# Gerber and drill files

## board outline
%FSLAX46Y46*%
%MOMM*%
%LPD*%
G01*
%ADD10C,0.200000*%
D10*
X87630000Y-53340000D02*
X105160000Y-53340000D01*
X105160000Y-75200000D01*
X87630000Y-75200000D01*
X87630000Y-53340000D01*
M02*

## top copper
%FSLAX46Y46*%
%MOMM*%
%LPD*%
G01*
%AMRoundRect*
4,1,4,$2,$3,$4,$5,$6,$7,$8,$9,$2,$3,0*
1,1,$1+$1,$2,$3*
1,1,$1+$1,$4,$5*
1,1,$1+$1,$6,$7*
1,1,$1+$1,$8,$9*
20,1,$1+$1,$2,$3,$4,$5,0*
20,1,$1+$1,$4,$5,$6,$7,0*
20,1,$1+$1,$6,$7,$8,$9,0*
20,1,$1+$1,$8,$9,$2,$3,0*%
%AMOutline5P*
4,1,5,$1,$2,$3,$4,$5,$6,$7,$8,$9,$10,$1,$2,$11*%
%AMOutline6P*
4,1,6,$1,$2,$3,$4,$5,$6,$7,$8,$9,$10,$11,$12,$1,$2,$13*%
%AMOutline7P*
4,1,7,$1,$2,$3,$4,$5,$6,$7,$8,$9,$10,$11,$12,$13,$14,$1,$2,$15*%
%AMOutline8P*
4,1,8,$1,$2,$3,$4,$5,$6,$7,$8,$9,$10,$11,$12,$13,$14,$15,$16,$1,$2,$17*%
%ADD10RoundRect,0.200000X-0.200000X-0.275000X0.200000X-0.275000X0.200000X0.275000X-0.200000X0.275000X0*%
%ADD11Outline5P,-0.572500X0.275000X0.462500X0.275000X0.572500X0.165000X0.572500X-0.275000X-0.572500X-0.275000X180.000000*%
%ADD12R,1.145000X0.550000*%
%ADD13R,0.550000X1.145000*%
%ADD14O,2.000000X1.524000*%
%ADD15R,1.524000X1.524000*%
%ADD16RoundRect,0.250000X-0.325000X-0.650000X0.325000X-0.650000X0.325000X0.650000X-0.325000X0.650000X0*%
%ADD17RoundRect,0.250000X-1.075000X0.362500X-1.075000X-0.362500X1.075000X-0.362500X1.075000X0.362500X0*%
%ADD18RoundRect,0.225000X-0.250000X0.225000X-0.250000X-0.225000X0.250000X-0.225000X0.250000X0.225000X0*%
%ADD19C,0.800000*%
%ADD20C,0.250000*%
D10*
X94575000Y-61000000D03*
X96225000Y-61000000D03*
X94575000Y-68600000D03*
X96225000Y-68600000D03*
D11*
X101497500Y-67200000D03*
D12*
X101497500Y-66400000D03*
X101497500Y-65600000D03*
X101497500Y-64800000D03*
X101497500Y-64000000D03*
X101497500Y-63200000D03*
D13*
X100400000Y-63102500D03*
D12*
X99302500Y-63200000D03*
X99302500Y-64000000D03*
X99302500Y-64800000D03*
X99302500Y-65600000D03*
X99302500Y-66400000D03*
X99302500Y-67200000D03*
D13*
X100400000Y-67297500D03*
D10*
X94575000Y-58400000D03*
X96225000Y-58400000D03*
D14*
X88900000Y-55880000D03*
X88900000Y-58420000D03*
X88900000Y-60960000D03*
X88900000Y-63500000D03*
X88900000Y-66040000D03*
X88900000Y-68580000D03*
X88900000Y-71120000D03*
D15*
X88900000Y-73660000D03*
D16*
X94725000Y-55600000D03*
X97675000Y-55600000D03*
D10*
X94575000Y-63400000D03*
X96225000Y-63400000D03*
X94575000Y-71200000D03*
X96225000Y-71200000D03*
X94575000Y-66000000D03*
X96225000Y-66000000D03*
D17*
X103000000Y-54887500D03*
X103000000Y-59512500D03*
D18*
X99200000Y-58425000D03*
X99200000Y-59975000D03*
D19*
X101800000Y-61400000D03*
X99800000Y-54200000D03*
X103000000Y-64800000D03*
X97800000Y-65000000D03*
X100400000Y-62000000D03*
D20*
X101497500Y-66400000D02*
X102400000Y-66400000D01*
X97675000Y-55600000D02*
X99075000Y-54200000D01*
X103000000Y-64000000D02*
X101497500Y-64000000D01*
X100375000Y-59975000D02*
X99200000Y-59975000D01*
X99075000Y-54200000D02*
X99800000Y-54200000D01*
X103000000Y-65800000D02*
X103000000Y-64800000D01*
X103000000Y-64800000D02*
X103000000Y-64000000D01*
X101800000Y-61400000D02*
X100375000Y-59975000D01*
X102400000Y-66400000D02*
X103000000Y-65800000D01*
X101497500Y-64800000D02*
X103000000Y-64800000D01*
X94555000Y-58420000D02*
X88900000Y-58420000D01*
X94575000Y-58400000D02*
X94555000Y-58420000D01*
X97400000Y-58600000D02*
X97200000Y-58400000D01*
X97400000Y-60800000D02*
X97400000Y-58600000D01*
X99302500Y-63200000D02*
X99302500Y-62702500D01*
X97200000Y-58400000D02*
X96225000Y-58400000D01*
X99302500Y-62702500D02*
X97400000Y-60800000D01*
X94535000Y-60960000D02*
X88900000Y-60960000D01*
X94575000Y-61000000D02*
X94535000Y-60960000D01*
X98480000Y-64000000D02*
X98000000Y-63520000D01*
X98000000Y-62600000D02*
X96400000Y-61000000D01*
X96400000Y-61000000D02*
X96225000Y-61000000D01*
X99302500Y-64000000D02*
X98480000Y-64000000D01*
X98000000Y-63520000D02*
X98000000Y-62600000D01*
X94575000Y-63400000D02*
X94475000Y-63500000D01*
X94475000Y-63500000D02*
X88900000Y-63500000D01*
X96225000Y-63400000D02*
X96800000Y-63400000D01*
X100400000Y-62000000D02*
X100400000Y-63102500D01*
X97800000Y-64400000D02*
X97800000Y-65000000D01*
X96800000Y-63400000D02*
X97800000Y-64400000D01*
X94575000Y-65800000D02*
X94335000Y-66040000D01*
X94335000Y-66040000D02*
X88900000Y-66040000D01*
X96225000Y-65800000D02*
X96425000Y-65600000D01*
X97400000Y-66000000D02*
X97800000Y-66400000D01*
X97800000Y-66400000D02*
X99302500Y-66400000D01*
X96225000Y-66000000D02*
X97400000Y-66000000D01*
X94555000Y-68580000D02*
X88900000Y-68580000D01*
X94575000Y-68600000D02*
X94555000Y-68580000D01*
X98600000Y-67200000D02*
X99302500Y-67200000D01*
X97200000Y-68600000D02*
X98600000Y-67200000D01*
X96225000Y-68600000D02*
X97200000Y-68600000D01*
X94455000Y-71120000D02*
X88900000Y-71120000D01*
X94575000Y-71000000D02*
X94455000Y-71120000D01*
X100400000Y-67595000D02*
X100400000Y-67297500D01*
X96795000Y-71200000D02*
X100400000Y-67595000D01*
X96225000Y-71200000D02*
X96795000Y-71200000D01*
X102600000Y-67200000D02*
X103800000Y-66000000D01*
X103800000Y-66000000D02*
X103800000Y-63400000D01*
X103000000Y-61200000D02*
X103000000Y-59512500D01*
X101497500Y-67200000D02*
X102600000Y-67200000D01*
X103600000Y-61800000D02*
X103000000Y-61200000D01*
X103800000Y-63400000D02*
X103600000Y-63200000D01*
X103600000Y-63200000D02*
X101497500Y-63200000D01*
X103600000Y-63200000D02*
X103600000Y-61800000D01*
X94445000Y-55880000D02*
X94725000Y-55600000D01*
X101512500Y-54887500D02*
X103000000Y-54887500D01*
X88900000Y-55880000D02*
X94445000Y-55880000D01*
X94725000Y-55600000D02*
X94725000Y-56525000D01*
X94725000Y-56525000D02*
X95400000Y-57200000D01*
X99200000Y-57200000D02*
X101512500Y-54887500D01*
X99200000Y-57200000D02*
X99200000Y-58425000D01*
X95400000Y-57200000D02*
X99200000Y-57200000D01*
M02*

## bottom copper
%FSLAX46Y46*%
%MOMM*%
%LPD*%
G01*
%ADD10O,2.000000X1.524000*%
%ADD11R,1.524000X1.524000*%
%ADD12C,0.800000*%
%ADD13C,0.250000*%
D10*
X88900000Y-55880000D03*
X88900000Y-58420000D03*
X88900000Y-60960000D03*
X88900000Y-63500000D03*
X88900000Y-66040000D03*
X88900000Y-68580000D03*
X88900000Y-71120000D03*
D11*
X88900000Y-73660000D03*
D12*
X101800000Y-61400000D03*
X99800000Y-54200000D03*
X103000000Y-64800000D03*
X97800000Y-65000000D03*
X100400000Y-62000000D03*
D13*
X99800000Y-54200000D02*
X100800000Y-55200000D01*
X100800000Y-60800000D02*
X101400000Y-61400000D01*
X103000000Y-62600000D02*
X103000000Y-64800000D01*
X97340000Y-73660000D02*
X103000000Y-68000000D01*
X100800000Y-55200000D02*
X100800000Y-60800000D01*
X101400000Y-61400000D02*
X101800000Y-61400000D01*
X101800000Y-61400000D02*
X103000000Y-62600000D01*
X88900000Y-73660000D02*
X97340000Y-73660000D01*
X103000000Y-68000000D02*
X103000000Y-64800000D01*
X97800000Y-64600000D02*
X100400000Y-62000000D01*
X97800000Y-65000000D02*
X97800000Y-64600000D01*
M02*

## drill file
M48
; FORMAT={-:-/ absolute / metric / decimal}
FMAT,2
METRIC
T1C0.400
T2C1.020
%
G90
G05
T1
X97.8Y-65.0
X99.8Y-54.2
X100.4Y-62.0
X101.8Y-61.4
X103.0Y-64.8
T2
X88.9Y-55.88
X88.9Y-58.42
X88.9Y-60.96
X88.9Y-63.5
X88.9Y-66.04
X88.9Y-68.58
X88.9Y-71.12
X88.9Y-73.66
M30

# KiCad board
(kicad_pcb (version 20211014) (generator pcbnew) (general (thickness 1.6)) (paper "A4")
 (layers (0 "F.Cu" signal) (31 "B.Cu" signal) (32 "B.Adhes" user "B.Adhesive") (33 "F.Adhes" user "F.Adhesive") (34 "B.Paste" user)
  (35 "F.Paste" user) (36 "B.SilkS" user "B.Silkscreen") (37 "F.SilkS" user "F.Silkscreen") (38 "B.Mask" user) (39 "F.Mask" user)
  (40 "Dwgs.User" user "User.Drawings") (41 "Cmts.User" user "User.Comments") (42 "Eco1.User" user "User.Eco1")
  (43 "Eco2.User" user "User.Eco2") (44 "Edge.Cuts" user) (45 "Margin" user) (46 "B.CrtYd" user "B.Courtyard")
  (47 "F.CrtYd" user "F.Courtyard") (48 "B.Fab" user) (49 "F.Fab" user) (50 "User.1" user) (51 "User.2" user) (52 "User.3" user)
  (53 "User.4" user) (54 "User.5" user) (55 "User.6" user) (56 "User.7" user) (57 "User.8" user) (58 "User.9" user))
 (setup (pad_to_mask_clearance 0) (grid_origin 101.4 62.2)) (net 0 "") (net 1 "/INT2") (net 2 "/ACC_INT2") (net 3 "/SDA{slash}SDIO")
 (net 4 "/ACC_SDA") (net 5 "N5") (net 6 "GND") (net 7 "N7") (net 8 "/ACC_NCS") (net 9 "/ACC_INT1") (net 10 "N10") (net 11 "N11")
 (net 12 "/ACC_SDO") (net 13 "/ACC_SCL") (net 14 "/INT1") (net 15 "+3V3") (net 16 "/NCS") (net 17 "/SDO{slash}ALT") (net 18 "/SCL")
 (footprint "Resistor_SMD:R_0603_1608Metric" (layer "F.Cu") (at 95.4 61)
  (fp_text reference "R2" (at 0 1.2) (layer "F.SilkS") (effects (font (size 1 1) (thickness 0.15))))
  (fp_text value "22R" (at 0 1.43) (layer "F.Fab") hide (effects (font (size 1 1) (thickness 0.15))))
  (pad "1" smd roundrect (at -0.825 0) (size 0.8 0.95) (layers "F.Cu" "F.Paste" "F.Mask") (roundrect_rratio 0.25) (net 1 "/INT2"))
  (pad "2" smd roundrect (at 0.825 0) (size 0.8 0.95) (layers "F.Cu" "F.Paste" "F.Mask") (roundrect_rratio 0.25) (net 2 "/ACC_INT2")))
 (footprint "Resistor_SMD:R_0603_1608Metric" (layer "F.Cu") (at 95.4 68.6)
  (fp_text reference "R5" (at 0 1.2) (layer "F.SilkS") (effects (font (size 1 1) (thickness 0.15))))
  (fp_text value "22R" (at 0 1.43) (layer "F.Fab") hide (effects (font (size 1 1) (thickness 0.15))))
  (pad "1" smd roundrect (at -0.825 0) (size 0.8 0.95) (layers "F.Cu" "F.Paste" "F.Mask") (roundrect_rratio 0.25) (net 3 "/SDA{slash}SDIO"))
  (pad "2" smd roundrect (at 0.825 0) (size 0.8 0.95) (layers "F.Cu" "F.Paste" "F.Mask") (roundrect_rratio 0.25) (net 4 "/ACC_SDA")))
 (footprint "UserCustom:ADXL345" (layer "F.Cu") (at 100.4 65.2 180)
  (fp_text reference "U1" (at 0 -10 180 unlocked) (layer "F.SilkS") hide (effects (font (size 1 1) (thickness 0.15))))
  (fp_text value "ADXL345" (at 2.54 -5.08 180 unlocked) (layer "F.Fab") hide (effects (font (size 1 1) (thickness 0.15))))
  (pad "1" smd roundrect (at -1.0975 -2 180) (size 1.145 0.55) (layers "F.Cu" "F.Paste" "F.Mask") (roundrect_rratio 0) (chamfer_ratio 0.2)
   (chamfer top_right) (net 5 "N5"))
  (pad "2" smd rect (at -1.0975 -1.2 180) (size 1.145 0.55) (layers "F.Cu" "F.Paste" "F.Mask") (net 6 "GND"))
  (pad "3" smd rect (at -1.0975 -0.4 180) (size 1.145 0.55) (layers "F.Cu" "F.Paste" "F.Mask") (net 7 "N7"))
  (pad "4" smd rect (at -1.0975 0.4 180) (size 1.145 0.55) (layers "F.Cu" "F.Paste" "F.Mask") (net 6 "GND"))
  (pad "5" smd rect (at -1.0975 1.2 180) (size 1.145 0.55) (layers "F.Cu" "F.Paste" "F.Mask") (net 6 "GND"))
  (pad "6" smd rect (at -1.0975 2 180) (size 1.145 0.55) (layers "F.Cu" "F.Paste" "F.Mask") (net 5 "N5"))
  (pad "7" smd rect (at 0 2.0975 180) (size 0.55 1.145) (layers "F.Cu" "F.Paste" "F.Mask") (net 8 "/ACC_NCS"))
  (pad "8" smd rect (at 1.0975 2 180) (size 1.145 0.55) (layers "F.Cu" "F.Paste" "F.Mask") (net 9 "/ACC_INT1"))
  (pad "9" smd rect (at 1.0975 1.2 180) (size 1.145 0.55) (layers "F.Cu" "F.Paste" "F.Mask") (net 2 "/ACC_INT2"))
  (pad "10" smd rect (at 1.0975 0.4 180) (size 1.145 0.55) (layers "F.Cu" "F.Paste" "F.Mask") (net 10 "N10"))
  (pad "11" smd rect (at 1.0975 -0.4 180) (size 1.145 0.55) (layers "F.Cu" "F.Paste" "F.Mask") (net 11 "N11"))
  (pad "12" smd rect (at 1.0975 -1.2 180) (size 1.145 0.55) (layers "F.Cu" "F.Paste" "F.Mask") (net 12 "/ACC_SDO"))
  (pad "13" smd rect (at 1.0975 -2 180) (size 1.145 0.55) (layers "F.Cu" "F.Paste" "F.Mask") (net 4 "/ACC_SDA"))
  (pad "14" smd rect (at 0 -2.0975 180) (size 0.55 1.145) (layers "F.Cu" "F.Paste" "F.Mask") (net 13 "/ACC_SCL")))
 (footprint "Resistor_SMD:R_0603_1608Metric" (layer "F.Cu") (at 95.4 58.4)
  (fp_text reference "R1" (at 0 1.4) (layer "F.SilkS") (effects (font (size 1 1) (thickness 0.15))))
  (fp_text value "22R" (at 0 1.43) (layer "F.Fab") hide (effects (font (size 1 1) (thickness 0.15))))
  (pad "1" smd roundrect (at -0.825 0) (size 0.8 0.95) (layers "F.Cu" "F.Paste" "F.Mask") (roundrect_rratio 0.25) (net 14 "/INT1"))
  (pad "2" smd roundrect (at 0.825 0) (size 0.8 0.95) (layers "F.Cu" "F.Paste" "F.Mask") (roundrect_rratio 0.25) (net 9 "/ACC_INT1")))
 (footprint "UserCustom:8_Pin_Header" (layer "F.Cu") (at 88.9 66.04)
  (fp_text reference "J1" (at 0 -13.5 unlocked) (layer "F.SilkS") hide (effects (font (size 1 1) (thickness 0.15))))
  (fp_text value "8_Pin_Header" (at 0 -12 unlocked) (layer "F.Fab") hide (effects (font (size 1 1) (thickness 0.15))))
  (pad "1" thru_hole oval (at 0 -10.16) (size 2 1.524) (drill 1.02) (layers *.Cu *.Mask) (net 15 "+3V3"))
  (pad "2" thru_hole oval (at 0 -7.62) (size 2 1.524) (drill 1.02) (layers *.Cu *.Mask) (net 14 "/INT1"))
  (pad "3" thru_hole oval (at 0 -5.08) (size 2 1.524) (drill 1.02) (layers *.Cu *.Mask) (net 1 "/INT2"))
  (pad "4" thru_hole oval (at 0 -2.54) (size 2 1.524) (drill 1.02) (layers *.Cu *.Mask) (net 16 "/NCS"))
  (pad "5" thru_hole oval (at 0 0) (size 2 1.524) (drill 1.02) (layers *.Cu *.Mask) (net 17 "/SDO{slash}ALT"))
  (pad "6" thru_hole oval (at 0 2.54) (size 2 1.524) (drill 1.02) (layers *.Cu *.Mask) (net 3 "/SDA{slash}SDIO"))
  (pad "7" thru_hole oval (at 0 5.08) (size 2 1.524) (drill 1.02) (layers *.Cu *.Mask) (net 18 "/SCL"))
  (pad "8" thru_hole rect (at 0 7.62) (size 1.524 1.524) (drill 1.02) (layers *.Cu *.Mask) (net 6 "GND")))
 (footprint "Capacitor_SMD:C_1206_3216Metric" (layer "F.Cu") (at 96.2 55.6)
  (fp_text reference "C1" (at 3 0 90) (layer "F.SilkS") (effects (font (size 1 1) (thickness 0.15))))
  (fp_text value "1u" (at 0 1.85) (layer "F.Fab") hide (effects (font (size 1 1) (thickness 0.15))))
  (pad "1" smd roundrect (at -1.475 0) (size 1.15 1.8) (layers "F.Cu" "F.Paste" "F.Mask") (roundrect_rratio 0.217391) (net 15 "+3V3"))
  (pad "2" smd roundrect (at 1.475 0) (size 1.15 1.8) (layers "F.Cu" "F.Paste" "F.Mask") (roundrect_rratio 0.217391) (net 6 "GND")))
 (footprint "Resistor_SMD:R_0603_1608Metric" (layer "F.Cu") (at 95.4 63.4)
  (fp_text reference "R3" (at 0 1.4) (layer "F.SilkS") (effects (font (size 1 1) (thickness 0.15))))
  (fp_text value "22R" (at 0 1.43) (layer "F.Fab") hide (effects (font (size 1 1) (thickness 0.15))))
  (pad "1" smd roundrect (at -0.825 0) (size 0.8 0.95) (layers "F.Cu" "F.Paste" "F.Mask") (roundrect_rratio 0.25) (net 16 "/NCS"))
  (pad "2" smd roundrect (at 0.825 0) (size 0.8 0.95) (layers "F.Cu" "F.Paste" "F.Mask") (roundrect_rratio 0.25) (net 8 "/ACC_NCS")))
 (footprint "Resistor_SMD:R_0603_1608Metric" (layer "F.Cu") (at 95.4 71.2)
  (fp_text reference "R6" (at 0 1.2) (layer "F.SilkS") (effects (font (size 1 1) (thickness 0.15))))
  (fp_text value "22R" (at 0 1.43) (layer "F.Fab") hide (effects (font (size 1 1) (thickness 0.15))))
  (pad "1" smd roundrect (at -0.825 0) (size 0.8 0.95) (layers "F.Cu" "F.Paste" "F.Mask") (roundrect_rratio 0.25) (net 18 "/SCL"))
  (pad "2" smd roundrect (at 0.825 0) (size 0.8 0.95) (layers "F.Cu" "F.Paste" "F.Mask") (roundrect_rratio 0.25) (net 13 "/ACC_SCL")))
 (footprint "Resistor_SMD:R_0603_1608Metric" (layer "F.Cu") (at 95.4 66)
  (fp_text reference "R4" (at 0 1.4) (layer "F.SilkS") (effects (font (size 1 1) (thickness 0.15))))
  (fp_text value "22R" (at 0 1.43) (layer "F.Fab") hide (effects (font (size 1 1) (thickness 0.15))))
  (pad "1" smd roundrect (at -0.825 0) (size 0.8 0.95) (layers "F.Cu" "F.Paste" "F.Mask") (roundrect_rratio 0.25) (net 17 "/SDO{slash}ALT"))
  (pad "2" smd roundrect (at 0.825 0) (size 0.8 0.95) (layers "F.Cu" "F.Paste" "F.Mask") (roundrect_rratio 0.25) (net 12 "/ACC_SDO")))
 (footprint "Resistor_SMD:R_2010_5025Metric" (layer "F.Cu") (at 103 57.2 -90)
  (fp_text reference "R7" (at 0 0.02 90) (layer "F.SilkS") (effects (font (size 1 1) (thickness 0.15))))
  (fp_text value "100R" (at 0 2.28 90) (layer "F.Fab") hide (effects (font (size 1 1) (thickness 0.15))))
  (pad "1" smd roundrect (at -2.3125 0 270) (size 1.225 2.65) (layers "F.Cu" "F.Paste" "F.Mask") (roundrect_rratio 0.204082) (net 15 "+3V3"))
  (pad "2" smd roundrect (at 2.3125 0 270) (size 1.225 2.65) (layers "F.Cu" "F.Paste" "F.Mask") (roundrect_rratio 0.204082) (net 5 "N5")))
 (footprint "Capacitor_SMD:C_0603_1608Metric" (layer "F.Cu") (at 99.2 59.2 -90)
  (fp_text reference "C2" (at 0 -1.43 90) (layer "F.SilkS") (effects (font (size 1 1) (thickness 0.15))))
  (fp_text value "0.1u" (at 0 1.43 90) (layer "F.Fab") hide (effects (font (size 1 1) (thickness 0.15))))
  (pad "1" smd roundrect (at -0.775 0 270) (size 0.9 0.95) (layers "F.Cu" "F.Paste" "F.Mask") (roundrect_rratio 0.25) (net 15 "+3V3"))
  (pad "2" smd roundrect (at 0.775 0 270) (size 0.9 0.95) (layers "F.Cu" "F.Paste" "F.Mask") (roundrect_rratio 0.25) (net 6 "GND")))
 (gr_rect (start 87.63 53.34) (end 105.16 75.2) (layer "Edge.Cuts") (width 0.2) (fill none))
 (segment (start 101.4975 66.4) (end 102.4 66.4) (width 0.25) (layer "F.Cu") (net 6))
 (segment (start 97.675 55.6) (end 99.075 54.2) (width 0.25) (layer "F.Cu") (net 6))
 (segment (start 103 64) (end 101.4975 64) (width 0.25) (layer "F.Cu") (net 6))
 (segment (start 100.375 59.975) (end 99.2 59.975) (width 0.25) (layer "F.Cu") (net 6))
 (segment (start 99.075 54.2) (end 99.8 54.2) (width 0.25) (layer "F.Cu") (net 6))
 (segment (start 103 65.8) (end 103 64.8) (width 0.25) (layer "F.Cu") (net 6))
 (segment (start 103 64.8) (end 103 64) (width 0.25) (layer "F.Cu") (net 6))
 (segment (start 101.8 61.4) (end 100.375 59.975) (width 0.25) (layer "F.Cu") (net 6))
 (segment (start 102.4 66.4) (end 103 65.8) (width 0.25) (layer "F.Cu") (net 6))
 (segment (start 101.4975 64.8) (end 103 64.8) (width 0.25) (layer "F.Cu") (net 6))
 (via (at 101.8 61.4) (size 0.8) (drill 0.4) (layers "F.Cu" "B.Cu") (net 6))
 (via (at 99.8 54.2) (size 0.8) (drill 0.4) (layers "F.Cu" "B.Cu") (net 6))
 (via (at 103 64.8) (size 0.8) (drill 0.4) (layers "F.Cu" "B.Cu") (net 6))
 (segment (start 99.8 54.2) (end 100.8 55.2) (width 0.25) (layer "B.Cu") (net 6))
 (segment (start 100.8 60.8) (end 101.4 61.4) (width 0.25) (layer "B.Cu") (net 6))
 (segment (start 103 62.6) (end 103 64.8) (width 0.25) (layer "B.Cu") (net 6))
 (segment (start 97.34 73.66) (end 103 68) (width 0.25) (layer "B.Cu") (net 6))
 (segment (start 100.8 55.2) (end 100.8 60.8) (width 0.25) (layer "B.Cu") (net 6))
 (segment (start 101.4 61.4) (end 101.8 61.4) (width 0.25) (layer "B.Cu") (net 6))
 (segment (start 101.8 61.4) (end 103 62.6) (width 0.25) (layer "B.Cu") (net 6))
 (segment (start 88.9 73.66) (end 97.34 73.66) (width 0.25) (layer "B.Cu") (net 6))
 (segment (start 103 68) (end 103 64.8) (width 0.25) (layer "B.Cu") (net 6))
 (segment (start 94.555 58.42) (end 88.9 58.42) (width 0.25) (layer "F.Cu") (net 14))
 (segment (start 94.575 58.4) (end 94.555 58.42) (width 0.25) (layer "F.Cu") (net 14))
 (segment (start 97.4 58.6) (end 97.2 58.4) (width 0.25) (layer "F.Cu") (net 9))
 (segment (start 97.4 60.8) (end 97.4 58.6) (width 0.25) (layer "F.Cu") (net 9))
 (segment (start 99.3025 63.2) (end 99.3025 62.7025) (width 0.25) (layer "F.Cu") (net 9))
 (segment (start 97.2 58.4) (end 96.225 58.4) (width 0.25) (layer "F.Cu") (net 9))
 (segment (start 99.3025 62.7025) (end 97.4 60.8) (width 0.25) (layer "F.Cu") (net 9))
 (segment (start 94.535 60.96) (end 88.9 60.96) (width 0.25) (layer "F.Cu") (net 1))
 (segment (start 94.575 61) (end 94.535 60.96) (width 0.25) (layer "F.Cu") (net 1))
 (segment (start 98.48 64) (end 98 63.52) (width 0.25) (layer "F.Cu") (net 2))
 (segment (start 98 62.6) (end 96.4 61) (width 0.25) (layer "F.Cu") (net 2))
 (segment (start 96.4 61) (end 96.225 61) (width 0.25) (layer "F.Cu") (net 2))
 (segment (start 99.3025 64) (end 98.48 64) (width 0.25) (layer "F.Cu") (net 2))
 (segment (start 98 63.52) (end 98 62.6) (width 0.25) (layer "F.Cu") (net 2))
 (segment (start 94.575 63.4) (end 94.475 63.5) (width 0.25) (layer "F.Cu") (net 16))
 (segment (start 94.475 63.5) (end 88.9 63.5) (width 0.25) (layer "F.Cu") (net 16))
 (segment (start 96.225 63.4) (end 96.8 63.4) (width 0.25) (layer "F.Cu") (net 8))
 (segment (start 100.4 62) (end 100.4 63.1025) (width 0.25) (layer "F.Cu") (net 8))
 (segment (start 97.8 64.4) (end 97.8 65) (width 0.25) (layer "F.Cu") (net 8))
 (segment (start 96.8 63.4) (end 97.8 64.4) (width 0.25) (layer "F.Cu") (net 8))
 (via (at 97.8 65) (size 0.8) (drill 0.4) (layers "F.Cu" "B.Cu") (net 8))
 (via (at 100.4 62) (size 0.8) (drill 0.4) (layers "F.Cu" "B.Cu") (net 8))
 (segment (start 97.8 64.6) (end 100.4 62) (width 0.25) (layer "B.Cu") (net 8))
 (segment (start 97.8 65) (end 97.8 64.6) (width 0.25) (layer "B.Cu") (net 8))
 (segment (start 94.575 65.8) (end 94.335 66.04) (width 0.25) (layer "F.Cu") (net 17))
 (segment (start 94.335 66.04) (end 88.9 66.04) (width 0.25) (layer "F.Cu") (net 17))
 (segment (start 96.225 65.8) (end 96.425 65.6) (width 0.25) (layer "F.Cu") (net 12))
 (segment (start 97.4 66) (end 97.8 66.4) (width 0.25) (layer "F.Cu") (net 12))
 (segment (start 97.8 66.4) (end 99.3025 66.4) (width 0.25) (layer "F.Cu") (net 12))
 (segment (start 96.225 66) (end 97.4 66) (width 0.25) (layer "F.Cu") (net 12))
 (segment (start 94.555 68.58) (end 88.9 68.58) (width 0.25) (layer "F.Cu") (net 3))
 (segment (start 94.575 68.6) (end 94.555 68.58) (width 0.25) (layer "F.Cu") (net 3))
 (segment (start 98.6 67.2) (end 99.3025 67.2) (width 0.25) (layer "F.Cu") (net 4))
 (segment (start 97.2 68.6) (end 98.6 67.2) (width 0.25) (layer "F.Cu") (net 4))
 (segment (start 96.225 68.6) (end 97.2 68.6) (width 0.25) (layer "F.Cu") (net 4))
 (segment (start 94.455 71.12) (end 88.9 71.12) (width 0.25) (layer "F.Cu") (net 18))
 (segment (start 94.575 71) (end 94.455 71.12) (width 0.25) (layer "F.Cu") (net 18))
 (segment (start 100.4 67.595) (end 100.4 67.2975) (width 0.25) (layer "F.Cu") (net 13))
 (segment (start 96.795 71.2) (end 100.4 67.595) (width 0.25) (layer "F.Cu") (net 13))
 (segment (start 96.225 71.2) (end 96.795 71.2) (width 0.25) (layer "F.Cu") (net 13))
 (segment (start 102.6 67.2) (end 103.8 66) (width 0.25) (layer "F.Cu") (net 5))
 (segment (start 103.8 66) (end 103.8 63.4) (width 0.25) (layer "F.Cu") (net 5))
 (segment (start 103 61.2) (end 103 59.5125) (width 0.25) (layer "F.Cu") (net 5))
 (segment (start 101.4975 67.2) (end 102.6 67.2) (width 0.25) (layer "F.Cu") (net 5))
 (segment (start 103.6 61.8) (end 103 61.2) (width 0.25) (layer "F.Cu") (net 5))
 (segment (start 103.8 63.4) (end 103.6 63.2) (width 0.25) (layer "F.Cu") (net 5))
 (segment (start 103.6 63.2) (end 101.4975 63.2) (width 0.25) (layer "F.Cu") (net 5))
 (segment (start 103.6 63.2) (end 103.6 61.8) (width 0.25) (layer "F.Cu") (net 5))
 (segment (start 94.445 55.88) (end 94.725 55.6) (width 0.25) (layer "F.Cu") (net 15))
 (segment (start 101.5125 54.8875) (end 103 54.8875) (width 0.25) (layer "F.Cu") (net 15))
 (segment (start 88.9 55.88) (end 94.445 55.88) (width 0.25) (layer "F.Cu") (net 15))
 (segment (start 94.725 55.6) (end 94.725 56.525) (width 0.25) (layer "F.Cu") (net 15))
 (segment (start 94.725 56.525) (end 95.4 57.2) (width 0.25) (layer "F.Cu") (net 15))
 (segment (start 99.2 57.2) (end 101.5125 54.8875) (width 0.25) (layer "F.Cu") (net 15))
 (segment (start 99.2 57.2) (end 99.2 58.425) (width 0.25) (layer "F.Cu") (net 15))
 (segment (start 95.4 57.2) (end 99.2 57.2) (width 0.25) (layer "F.Cu") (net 15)))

